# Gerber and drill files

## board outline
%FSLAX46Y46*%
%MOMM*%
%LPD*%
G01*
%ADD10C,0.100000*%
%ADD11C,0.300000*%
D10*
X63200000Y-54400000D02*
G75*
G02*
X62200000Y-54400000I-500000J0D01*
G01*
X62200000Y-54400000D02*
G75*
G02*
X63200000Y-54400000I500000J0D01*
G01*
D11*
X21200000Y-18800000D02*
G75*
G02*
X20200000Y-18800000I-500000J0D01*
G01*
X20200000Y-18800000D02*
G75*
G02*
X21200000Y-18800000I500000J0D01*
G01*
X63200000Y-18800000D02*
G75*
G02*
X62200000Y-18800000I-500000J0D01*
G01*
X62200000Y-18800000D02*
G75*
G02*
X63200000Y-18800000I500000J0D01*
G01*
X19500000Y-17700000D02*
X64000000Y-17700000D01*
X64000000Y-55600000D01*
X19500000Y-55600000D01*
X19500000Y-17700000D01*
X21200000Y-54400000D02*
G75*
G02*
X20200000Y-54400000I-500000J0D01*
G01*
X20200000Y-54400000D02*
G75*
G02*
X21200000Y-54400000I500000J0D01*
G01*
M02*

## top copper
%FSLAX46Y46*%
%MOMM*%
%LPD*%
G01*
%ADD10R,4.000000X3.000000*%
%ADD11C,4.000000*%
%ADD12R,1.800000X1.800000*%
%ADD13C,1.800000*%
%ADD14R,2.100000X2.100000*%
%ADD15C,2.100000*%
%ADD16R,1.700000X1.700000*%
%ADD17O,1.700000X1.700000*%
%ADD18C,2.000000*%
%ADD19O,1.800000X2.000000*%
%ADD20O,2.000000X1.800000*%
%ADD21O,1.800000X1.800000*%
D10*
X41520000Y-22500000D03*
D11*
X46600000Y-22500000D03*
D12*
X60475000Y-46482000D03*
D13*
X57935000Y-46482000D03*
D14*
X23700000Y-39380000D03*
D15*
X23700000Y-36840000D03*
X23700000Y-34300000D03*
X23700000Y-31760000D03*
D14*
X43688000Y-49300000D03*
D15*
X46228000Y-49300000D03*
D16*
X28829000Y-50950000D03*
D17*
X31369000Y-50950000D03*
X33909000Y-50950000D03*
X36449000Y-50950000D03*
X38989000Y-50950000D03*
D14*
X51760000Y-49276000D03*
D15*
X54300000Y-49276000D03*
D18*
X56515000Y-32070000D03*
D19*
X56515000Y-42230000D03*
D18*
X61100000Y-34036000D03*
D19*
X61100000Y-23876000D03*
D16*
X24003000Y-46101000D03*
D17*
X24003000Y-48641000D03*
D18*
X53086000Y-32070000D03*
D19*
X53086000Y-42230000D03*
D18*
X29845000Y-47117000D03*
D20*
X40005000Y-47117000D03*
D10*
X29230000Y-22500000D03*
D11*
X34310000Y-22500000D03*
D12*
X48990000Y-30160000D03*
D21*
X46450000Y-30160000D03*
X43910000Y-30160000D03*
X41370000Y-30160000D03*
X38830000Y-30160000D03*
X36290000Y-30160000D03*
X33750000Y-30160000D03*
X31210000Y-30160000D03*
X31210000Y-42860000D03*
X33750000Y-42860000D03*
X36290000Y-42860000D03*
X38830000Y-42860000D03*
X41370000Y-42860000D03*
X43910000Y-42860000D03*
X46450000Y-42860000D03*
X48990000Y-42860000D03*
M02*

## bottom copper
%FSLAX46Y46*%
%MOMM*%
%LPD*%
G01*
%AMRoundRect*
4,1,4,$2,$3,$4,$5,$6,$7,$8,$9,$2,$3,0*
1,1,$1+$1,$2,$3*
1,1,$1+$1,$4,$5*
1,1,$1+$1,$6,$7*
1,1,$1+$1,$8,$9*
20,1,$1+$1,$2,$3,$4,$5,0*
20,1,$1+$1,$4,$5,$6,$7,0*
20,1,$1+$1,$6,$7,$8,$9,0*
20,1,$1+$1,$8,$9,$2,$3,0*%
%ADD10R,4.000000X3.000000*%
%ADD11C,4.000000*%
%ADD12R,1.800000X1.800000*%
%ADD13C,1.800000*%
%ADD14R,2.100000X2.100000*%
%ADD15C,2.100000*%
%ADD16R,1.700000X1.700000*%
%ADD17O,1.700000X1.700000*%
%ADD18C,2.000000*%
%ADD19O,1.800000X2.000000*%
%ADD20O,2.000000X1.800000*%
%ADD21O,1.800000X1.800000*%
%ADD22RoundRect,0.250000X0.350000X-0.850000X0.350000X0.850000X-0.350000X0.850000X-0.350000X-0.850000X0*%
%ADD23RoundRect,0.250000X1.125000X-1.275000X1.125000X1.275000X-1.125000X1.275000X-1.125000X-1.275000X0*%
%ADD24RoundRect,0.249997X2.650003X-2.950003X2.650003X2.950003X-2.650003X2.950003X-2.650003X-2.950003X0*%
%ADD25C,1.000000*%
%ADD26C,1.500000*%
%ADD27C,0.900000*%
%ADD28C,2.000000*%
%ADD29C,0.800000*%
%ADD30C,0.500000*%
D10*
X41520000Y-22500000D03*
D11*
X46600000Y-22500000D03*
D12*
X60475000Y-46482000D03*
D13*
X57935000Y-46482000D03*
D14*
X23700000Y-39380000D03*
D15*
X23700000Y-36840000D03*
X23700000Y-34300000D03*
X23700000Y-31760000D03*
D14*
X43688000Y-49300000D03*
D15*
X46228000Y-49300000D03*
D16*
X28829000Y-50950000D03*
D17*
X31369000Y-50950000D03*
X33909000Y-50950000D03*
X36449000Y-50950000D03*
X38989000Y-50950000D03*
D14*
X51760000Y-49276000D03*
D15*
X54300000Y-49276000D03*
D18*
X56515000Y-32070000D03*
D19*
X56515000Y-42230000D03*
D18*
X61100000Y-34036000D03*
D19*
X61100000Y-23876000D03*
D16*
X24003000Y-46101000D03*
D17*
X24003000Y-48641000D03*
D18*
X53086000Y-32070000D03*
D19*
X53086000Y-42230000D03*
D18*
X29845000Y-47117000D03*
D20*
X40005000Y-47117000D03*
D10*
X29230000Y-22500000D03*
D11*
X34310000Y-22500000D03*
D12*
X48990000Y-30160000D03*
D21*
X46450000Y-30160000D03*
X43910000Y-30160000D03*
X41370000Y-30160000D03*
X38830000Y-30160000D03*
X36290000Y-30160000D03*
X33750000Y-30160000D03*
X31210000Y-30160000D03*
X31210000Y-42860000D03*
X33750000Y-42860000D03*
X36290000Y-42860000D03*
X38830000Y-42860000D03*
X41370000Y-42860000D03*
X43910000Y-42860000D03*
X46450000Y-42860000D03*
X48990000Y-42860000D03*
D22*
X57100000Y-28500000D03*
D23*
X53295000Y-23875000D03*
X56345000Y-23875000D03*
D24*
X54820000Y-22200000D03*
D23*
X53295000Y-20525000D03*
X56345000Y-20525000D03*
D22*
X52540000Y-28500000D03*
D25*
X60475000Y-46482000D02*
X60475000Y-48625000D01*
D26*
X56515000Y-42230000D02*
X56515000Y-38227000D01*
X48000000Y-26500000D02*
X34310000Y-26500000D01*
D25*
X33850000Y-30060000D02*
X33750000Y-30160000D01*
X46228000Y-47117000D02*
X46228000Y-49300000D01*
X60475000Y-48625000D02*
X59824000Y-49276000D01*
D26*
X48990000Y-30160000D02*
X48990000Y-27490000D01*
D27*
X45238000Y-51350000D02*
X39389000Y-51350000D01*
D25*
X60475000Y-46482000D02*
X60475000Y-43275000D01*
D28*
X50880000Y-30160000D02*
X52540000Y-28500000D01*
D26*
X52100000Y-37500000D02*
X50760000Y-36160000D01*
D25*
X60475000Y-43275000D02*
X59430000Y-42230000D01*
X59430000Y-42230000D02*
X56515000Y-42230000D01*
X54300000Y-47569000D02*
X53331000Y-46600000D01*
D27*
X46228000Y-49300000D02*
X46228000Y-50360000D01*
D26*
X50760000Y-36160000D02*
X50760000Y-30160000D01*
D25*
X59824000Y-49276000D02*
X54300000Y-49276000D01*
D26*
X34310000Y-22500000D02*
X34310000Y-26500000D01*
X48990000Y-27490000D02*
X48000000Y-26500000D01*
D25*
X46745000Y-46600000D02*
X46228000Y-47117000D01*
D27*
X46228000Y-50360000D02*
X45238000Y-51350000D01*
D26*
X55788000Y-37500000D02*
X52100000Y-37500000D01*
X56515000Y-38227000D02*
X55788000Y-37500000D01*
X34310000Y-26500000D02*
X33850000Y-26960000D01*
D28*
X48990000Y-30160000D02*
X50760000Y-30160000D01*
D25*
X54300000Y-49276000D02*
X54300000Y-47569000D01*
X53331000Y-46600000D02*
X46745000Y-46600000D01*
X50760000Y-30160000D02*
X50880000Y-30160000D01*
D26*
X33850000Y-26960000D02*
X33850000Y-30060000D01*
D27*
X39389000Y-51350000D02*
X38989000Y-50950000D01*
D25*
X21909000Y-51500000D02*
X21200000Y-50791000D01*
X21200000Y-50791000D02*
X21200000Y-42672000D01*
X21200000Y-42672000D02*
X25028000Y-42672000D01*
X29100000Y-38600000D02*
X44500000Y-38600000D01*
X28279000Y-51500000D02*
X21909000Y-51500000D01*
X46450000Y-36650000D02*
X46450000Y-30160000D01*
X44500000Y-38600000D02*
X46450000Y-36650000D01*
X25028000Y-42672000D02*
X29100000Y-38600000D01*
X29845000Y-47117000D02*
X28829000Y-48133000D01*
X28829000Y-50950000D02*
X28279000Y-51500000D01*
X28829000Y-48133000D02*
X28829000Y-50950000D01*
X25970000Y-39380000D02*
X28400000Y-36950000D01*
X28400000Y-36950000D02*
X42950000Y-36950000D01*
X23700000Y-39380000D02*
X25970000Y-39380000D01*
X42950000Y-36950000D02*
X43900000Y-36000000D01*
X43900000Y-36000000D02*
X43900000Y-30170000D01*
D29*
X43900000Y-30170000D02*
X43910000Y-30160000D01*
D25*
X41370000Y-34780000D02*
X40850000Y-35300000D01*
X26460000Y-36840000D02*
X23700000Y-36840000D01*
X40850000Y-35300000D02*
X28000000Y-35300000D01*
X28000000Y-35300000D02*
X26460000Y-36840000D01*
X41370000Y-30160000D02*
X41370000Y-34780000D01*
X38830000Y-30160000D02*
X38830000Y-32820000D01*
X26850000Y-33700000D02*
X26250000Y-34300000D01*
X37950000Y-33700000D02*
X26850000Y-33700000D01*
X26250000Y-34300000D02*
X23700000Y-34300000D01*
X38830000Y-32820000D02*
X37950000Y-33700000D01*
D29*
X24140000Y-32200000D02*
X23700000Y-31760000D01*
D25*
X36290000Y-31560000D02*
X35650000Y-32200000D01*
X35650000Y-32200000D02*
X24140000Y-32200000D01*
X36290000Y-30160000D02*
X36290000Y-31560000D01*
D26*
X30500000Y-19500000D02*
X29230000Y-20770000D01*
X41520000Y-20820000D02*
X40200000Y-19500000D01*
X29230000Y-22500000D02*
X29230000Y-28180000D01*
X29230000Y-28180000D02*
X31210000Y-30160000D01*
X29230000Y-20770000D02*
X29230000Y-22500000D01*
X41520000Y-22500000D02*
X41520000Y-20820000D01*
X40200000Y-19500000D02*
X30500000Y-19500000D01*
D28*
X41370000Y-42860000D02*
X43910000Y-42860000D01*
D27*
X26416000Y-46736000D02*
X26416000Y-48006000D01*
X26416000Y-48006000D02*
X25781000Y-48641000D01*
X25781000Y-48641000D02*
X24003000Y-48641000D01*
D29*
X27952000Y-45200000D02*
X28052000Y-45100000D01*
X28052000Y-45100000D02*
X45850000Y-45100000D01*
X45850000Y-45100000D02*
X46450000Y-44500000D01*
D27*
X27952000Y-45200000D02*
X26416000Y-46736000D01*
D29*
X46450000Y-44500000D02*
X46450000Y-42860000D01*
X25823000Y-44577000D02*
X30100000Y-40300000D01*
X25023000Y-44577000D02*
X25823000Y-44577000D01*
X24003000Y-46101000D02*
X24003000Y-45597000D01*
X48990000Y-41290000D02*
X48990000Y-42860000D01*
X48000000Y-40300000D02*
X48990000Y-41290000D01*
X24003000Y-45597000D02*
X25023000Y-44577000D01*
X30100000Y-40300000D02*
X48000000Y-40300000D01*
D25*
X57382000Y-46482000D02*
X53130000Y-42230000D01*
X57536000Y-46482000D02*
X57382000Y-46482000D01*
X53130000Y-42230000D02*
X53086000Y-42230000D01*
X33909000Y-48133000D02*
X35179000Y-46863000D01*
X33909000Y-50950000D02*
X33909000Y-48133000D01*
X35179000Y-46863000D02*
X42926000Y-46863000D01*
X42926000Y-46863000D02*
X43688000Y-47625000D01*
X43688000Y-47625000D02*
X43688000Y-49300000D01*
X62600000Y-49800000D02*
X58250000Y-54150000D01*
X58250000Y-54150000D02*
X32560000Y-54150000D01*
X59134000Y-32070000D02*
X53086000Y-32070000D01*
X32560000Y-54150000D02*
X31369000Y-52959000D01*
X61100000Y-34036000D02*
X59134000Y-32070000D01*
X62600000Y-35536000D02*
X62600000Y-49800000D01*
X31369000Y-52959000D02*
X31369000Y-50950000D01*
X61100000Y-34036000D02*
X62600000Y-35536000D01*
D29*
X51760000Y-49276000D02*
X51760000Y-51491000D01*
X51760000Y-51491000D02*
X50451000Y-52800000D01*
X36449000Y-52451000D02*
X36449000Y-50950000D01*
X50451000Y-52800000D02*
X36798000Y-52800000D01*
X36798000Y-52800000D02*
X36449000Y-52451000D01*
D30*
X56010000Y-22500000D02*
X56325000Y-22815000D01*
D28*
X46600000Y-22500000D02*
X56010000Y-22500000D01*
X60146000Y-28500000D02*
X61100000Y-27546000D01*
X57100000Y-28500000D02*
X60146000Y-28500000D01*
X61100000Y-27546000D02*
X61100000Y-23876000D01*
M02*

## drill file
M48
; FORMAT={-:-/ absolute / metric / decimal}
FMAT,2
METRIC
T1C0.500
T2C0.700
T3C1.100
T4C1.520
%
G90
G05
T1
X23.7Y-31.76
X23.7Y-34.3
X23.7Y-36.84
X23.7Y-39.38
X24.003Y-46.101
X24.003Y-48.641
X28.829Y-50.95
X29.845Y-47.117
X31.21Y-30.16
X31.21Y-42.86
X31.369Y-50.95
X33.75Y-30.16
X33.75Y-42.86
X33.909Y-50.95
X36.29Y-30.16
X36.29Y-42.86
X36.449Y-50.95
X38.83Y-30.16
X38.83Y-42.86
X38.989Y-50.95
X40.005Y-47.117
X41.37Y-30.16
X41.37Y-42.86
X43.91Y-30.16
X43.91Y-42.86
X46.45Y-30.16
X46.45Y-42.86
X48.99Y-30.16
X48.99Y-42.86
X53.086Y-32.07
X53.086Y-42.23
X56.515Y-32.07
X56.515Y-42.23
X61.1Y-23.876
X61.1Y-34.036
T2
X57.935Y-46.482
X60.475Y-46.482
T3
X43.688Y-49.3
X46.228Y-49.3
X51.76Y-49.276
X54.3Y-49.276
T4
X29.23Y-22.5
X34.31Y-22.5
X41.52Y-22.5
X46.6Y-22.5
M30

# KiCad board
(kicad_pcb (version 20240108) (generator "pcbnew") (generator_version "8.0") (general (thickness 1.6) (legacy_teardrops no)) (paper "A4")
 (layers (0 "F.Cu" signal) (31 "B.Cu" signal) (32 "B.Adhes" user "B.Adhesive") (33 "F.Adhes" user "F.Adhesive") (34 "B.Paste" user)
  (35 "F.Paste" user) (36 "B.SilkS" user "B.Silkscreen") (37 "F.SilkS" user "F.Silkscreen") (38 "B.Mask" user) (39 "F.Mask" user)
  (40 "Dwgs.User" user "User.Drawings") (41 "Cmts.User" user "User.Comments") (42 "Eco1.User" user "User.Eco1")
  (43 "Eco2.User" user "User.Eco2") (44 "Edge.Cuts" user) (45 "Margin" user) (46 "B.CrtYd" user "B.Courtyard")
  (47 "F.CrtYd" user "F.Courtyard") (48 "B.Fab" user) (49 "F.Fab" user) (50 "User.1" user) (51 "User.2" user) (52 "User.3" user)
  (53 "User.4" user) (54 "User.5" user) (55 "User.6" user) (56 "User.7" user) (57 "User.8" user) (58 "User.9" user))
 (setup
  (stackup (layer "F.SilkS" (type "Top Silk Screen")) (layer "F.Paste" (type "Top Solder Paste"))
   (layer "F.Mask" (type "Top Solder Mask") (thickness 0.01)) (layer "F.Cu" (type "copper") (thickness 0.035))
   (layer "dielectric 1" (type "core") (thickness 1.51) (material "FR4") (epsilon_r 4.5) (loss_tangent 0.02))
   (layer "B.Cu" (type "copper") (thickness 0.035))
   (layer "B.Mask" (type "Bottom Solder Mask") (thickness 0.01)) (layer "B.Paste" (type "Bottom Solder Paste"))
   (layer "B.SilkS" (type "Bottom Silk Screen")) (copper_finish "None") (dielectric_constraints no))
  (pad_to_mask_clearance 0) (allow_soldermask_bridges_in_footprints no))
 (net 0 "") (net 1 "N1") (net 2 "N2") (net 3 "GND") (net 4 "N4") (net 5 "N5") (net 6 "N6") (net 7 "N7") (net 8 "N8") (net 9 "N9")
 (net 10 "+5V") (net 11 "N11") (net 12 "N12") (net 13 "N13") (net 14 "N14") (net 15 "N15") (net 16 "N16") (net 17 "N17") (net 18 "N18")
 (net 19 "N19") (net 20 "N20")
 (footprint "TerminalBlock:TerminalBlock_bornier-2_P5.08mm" (layer "F.Cu") (at 41.52 22.5)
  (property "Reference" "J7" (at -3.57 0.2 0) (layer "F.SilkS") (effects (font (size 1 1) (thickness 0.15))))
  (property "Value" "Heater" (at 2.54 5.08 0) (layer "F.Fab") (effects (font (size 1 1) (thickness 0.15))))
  (pad "1" thru_hole rect (at 0 0) (size 4 3) (drill 1.52) (layers "*.Cu" "*.Mask") (remove_unused_layers no) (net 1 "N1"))
  (pad "2" thru_hole circle (at 5.08 0) (size 4 3) (drill 1.52) (layers "*.Cu" "*.Mask") (remove_unused_layers no) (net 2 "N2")))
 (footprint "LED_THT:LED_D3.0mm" (layer "F.Cu") (at 60.475 46.482 180)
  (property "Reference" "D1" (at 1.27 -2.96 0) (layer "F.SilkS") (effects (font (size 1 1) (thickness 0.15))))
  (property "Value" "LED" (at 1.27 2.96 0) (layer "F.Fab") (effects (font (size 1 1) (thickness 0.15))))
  (pad "1" thru_hole rect (at 0 0 180) (size 1.8 1.8) (drill 0.7) (layers "*.Cu" "*.Mask") (remove_unused_layers no) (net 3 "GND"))
  (pad "2" thru_hole circle (at 2.54 0 180) (size 1.8 1.8) (drill 0.7) (layers "*.Cu" "*.Mask") (remove_unused_layers no) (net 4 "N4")))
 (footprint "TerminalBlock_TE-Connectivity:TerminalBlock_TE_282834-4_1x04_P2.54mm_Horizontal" (layer "F.Cu") (at 23.7 39.38 90)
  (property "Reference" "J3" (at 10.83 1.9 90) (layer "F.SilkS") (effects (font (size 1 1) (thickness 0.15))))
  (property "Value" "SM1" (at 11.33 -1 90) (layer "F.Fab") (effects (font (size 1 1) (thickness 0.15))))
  (pad "1" thru_hole rect (at 0 0 90) (size 2.1 2.1) (drill 0.5) (layers "*.Cu" "*.Mask") (remove_unused_layers no) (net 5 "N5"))
  (pad "2" thru_hole circle (at 2.54 0 90) (size 2.1 2.1) (drill 0.5) (layers "*.Cu" "*.Mask") (remove_unused_layers no) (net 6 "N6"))
  (pad "3" thru_hole circle (at 5.08 0 90) (size 2.1 2.1) (drill 0.5) (layers "*.Cu" "*.Mask") (remove_unused_layers no) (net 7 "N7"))
  (pad "4" thru_hole circle (at 7.62 0 90) (size 2.1 2.1) (drill 0.5) (layers "*.Cu" "*.Mask") (remove_unused_layers no) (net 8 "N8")))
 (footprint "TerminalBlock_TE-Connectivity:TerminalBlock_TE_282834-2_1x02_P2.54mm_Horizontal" (layer "F.Cu") (at 43.688 49.3)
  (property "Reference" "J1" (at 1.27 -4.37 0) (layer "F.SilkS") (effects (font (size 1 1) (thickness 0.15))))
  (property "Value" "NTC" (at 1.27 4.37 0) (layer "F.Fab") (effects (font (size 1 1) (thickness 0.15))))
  (pad "1" thru_hole rect (at 0 0) (size 2.1 2.1) (drill 1.1) (layers "*.Cu" "*.Mask") (remove_unused_layers no) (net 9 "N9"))
  (pad "2" thru_hole circle (at 2.54 0) (size 2.1 2.1) (drill 1.1) (layers "*.Cu" "*.Mask") (remove_unused_layers no) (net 3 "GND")))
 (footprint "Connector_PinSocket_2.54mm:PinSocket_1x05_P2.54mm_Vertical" (layer "F.Cu") (at 28.829 50.95 90)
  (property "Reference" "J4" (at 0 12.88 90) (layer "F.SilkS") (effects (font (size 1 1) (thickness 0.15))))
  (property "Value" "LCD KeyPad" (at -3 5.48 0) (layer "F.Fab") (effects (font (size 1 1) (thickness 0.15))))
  (pad "1" thru_hole rect (at 0 0 90) (size 1.7 1.7) (drill 0.5) (layers "*.Cu" "*.Mask") (remove_unused_layers no) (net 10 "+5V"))
  (pad "2" thru_hole oval (at 0 2.54 90) (size 1.7 1.7) (drill 0.5) (layers "*.Cu" "*.Mask") (remove_unused_layers no) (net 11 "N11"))
  (pad "3" thru_hole oval (at 0 5.08 90) (size 1.7 1.7) (drill 0.5) (layers "*.Cu" "*.Mask") (remove_unused_layers no) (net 9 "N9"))
  (pad "4" thru_hole oval (at 0 7.62 90) (size 1.7 1.7) (drill 0.5) (layers "*.Cu" "*.Mask") (remove_unused_layers no) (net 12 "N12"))
  (pad "5" thru_hole oval (at 0 10.16 90) (size 1.7 1.7) (drill 0.5) (layers "*.Cu" "*.Mask") (remove_unused_layers no) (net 3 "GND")))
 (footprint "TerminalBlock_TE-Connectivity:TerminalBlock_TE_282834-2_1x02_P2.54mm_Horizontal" (layer "F.Cu") (at 51.76 49.276)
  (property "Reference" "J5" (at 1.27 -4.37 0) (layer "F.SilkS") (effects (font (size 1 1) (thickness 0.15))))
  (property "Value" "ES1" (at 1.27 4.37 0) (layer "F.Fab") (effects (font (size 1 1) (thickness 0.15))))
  (pad "1" thru_hole rect (at 0 0) (size 2.1 2.1) (drill 1.1) (layers "*.Cu" "*.Mask") (remove_unused_layers no) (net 12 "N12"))
  (pad "2" thru_hole circle (at 2.54 0) (size 2.1 2.1) (drill 1.1) (layers "*.Cu" "*.Mask") (remove_unused_layers no) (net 3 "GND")))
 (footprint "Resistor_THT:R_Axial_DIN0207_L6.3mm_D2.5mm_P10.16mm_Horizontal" (layer "F.Cu") (at 56.515 32.07 -90)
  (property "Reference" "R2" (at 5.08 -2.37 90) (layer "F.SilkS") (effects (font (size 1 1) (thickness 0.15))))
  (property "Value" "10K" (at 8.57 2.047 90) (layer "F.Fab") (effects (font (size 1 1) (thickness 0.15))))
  (pad "1" thru_hole circle (at 0 0 270) (size 2 1.6) (drill 0.5) (layers "*.Cu" "*.Mask") (remove_unused_layers no) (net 11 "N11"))
  (pad "2" thru_hole oval (at 10.16 0 270) (size 2 1.8) (drill 0.5) (layers "*.Cu" "*.Mask") (remove_unused_layers no) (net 3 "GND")))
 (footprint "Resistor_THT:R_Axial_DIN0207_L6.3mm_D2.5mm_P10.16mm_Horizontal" (layer "F.Cu") (at 61.1 34.036 90)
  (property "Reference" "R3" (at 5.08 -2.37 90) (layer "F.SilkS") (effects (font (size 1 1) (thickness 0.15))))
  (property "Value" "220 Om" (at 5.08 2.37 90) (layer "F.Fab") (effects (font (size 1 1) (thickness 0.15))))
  (pad "1" thru_hole circle (at 0 0 90) (size 2 1.6) (drill 0.5) (layers "*.Cu" "*.Mask") (remove_unused_layers no) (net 11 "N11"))
  (pad "2" thru_hole oval (at 10.16 0 90) (size 2 1.8) (drill 0.5) (layers "*.Cu" "*.Mask") (remove_unused_layers no) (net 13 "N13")))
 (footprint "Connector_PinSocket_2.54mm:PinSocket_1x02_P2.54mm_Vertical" (layer "F.Cu") (at 24.003 46.101)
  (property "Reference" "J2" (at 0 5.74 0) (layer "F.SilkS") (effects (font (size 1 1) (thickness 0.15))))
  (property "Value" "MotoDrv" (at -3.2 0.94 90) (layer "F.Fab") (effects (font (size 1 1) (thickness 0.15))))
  (pad "1" thru_hole rect (at 0 0) (size 1.7 1.7) (drill 0.5) (layers "*.Cu" "*.Mask") (remove_unused_layers no) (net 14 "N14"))
  (pad "2" thru_hole oval (at 0 2.54) (size 1.7 1.7) (drill 0.5) (layers "*.Cu" "*.Mask") (remove_unused_layers no) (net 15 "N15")))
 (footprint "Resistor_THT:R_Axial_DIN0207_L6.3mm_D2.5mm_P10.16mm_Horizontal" (layer "F.Cu") (at 53.086 32.07 -90)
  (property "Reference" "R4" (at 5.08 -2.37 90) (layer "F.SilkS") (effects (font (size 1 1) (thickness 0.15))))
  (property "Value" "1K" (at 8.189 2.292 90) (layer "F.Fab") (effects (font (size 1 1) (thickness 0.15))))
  (pad "1" thru_hole circle (at 0 0 270) (size 2 1.6) (drill 0.5) (layers "*.Cu" "*.Mask") (remove_unused_layers no) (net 11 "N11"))
  (pad "2" thru_hole oval (at 10.16 0 270) (size 2 1.8) (drill 0.5) (layers "*.Cu" "*.Mask") (remove_unused_layers no) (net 4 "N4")))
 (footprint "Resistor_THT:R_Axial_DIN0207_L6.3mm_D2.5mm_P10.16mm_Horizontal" (layer "F.Cu") (at 29.845 47.117)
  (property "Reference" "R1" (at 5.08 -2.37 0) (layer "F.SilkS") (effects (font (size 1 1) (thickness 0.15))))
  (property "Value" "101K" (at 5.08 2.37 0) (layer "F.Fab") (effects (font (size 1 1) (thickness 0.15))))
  (pad "1" thru_hole circle (at 0 0) (size 2 1.6) (drill 0.5) (layers "*.Cu" "*.Mask") (remove_unused_layers no) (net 10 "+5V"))
  (pad "2" thru_hole oval (at 10.16 0) (size 2 1.8) (drill 0.5) (layers "*.Cu" "*.Mask") (remove_unused_layers no) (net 9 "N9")))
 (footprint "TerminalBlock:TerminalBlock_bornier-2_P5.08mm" (layer "F.Cu") (at 29.23 22.5)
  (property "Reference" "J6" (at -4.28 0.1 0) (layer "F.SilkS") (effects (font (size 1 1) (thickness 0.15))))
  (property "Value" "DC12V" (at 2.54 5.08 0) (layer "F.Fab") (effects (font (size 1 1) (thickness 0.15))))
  (pad "1" thru_hole rect (at 0 0) (size 4 3) (drill 1.52) (layers "*.Cu" "*.Mask") (remove_unused_layers no) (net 1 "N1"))
  (pad "2" thru_hole circle (at 5.08 0) (size 4 3) (drill 1.52) (layers "*.Cu" "*.Mask") (remove_unused_layers no) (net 3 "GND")))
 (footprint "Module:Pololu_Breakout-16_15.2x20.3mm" (layer "F.Cu") (at 48.99 30.16 -90)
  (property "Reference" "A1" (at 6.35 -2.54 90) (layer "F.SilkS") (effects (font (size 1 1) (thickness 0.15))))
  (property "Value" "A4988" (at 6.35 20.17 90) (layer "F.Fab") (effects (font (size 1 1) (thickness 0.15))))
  (pad "1" thru_hole rect (at 0 0 270) (size 1.8 1.8) (drill 0.5) (layers "*.Cu" "*.Mask") (remove_unused_layers no) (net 3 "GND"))
  (pad "2" thru_hole oval (at 0 2.54 270) (size 1.8 1.8) (drill 0.5) (layers "*.Cu" "*.Mask") (remove_unused_layers no) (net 10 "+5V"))
  (pad "3" thru_hole oval (at 0 5.08 270) (size 1.8 1.8) (drill 0.5) (layers "*.Cu" "*.Mask") (remove_unused_layers no) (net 5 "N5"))
  (pad "4" thru_hole oval (at 0 7.62 270) (size 1.8 1.8) (drill 0.5) (layers "*.Cu" "*.Mask") (remove_unused_layers no) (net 6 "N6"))
  (pad "5" thru_hole oval (at 0 10.16 270) (size 1.8 1.8) (drill 0.5) (layers "*.Cu" "*.Mask") (remove_unused_layers no) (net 7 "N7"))
  (pad "6" thru_hole oval (at 0 12.7 270) (size 1.8 1.8) (drill 0.5) (layers "*.Cu" "*.Mask") (remove_unused_layers no) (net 8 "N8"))
  (pad "7" thru_hole oval (at 0 15.24 270) (size 1.8 1.8) (drill 0.5) (layers "*.Cu" "*.Mask") (remove_unused_layers no) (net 3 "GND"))
  (pad "8" thru_hole oval (at 0 17.78 270) (size 1.8 1.8) (drill 0.5) (layers "*.Cu" "*.Mask") (remove_unused_layers no) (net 1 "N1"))
  (pad "9" thru_hole oval (at 12.7 17.78 270) (size 1.8 1.8) (drill 0.5) (layers "*.Cu" "*.Mask") (remove_unused_layers no) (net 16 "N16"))
  (pad "10" thru_hole oval (at 12.7 15.24 270) (size 1.8 1.8) (drill 0.5) (layers "*.Cu" "*.Mask") (remove_unused_layers no) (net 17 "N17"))
  (pad "11" thru_hole oval (at 12.7 12.7 270) (size 1.8 1.8) (drill 0.5) (layers "*.Cu" "*.Mask") (remove_unused_layers no) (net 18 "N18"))
  (pad "12" thru_hole oval (at 12.7 10.16 270) (size 1.8 1.8) (drill 0.5) (layers "*.Cu" "*.Mask") (remove_unused_layers no) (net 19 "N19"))
  (pad "13" thru_hole oval (at 12.7 7.62 270) (size 1.8 1.8) (drill 0.5) (layers "*.Cu" "*.Mask") (remove_unused_layers no) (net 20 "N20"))
  (pad "14" thru_hole oval (at 12.7 5.08 270) (size 1.8 1.8) (drill 0.5) (layers "*.Cu" "*.Mask") (remove_unused_layers no) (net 20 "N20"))
  (pad "15" thru_hole oval (at 12.7 2.54 270) (size 1.8 1.8) (drill 0.5) (layers "*.Cu" "*.Mask") (remove_unused_layers no) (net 15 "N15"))
  (pad "16" thru_hole oval (at 12.7 0 270) (size 1.8 1.8) (drill 0.5) (layers "*.Cu" "*.Mask") (remove_unused_layers no) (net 14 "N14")))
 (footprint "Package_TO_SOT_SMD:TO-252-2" (layer "B.Cu") (at 54.82 23.46 90)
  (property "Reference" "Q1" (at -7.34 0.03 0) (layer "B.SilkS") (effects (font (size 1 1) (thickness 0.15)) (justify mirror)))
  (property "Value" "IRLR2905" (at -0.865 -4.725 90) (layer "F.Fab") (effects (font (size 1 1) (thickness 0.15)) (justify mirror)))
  (pad "1" smd roundrect (at -5.04 2.28 90) (size 2.2 1.2) (layers "B.Cu" "B.Paste" "B.Mask") (roundrect_rratio 0.208333) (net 13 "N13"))
  (pad "2" smd roundrect (at -0.415 -1.525 90) (size 3.05 2.75) (layers "B.Cu" "B.Paste") (roundrect_rratio 0.090909) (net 2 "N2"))
  (pad "2" smd roundrect (at -0.415 1.525 90) (size 3.05 2.75) (layers "B.Cu" "B.Paste") (roundrect_rratio 0.090909) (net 2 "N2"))
  (pad "2" smd roundrect (at 1.26 0 90) (size 6.4 5.8) (layers "B.Cu" "B.Mask") (roundrect_rratio 0.043103) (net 2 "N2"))
  (pad "2" smd roundrect (at 2.935 -1.525 90) (size 3.05 2.75) (layers "B.Cu" "B.Paste") (roundrect_rratio 0.090909) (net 2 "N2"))
  (pad "2" smd roundrect (at 2.935 1.525 90) (size 3.05 2.75) (layers "B.Cu" "B.Paste") (roundrect_rratio 0.090909) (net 2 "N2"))
  (pad "3" smd roundrect (at -5.04 -2.28 90) (size 2.2 1.2) (layers "B.Cu" "B.Paste" "B.Mask") (roundrect_rratio 0.208333) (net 3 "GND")))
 (gr_circle (center 62.7 54.4) (end 63.2 54.4) (stroke (width 0.1) (type default)) (fill none) (layer "Edge.Cuts"))
 (gr_circle (center 20.7 18.8) (end 21.2 18.8) (stroke (width 0.3) (type default)) (fill none) (layer "Edge.Cuts"))
 (gr_circle (center 62.7 18.8) (end 63.2 18.8) (stroke (width 0.3) (type default)) (fill none) (layer "Edge.Cuts"))
 (gr_rect (start 19.5 17.7) (end 64 55.6) (stroke (width 0.3) (type default)) (fill none) (layer "Edge.Cuts"))
 (gr_circle (center 20.7 54.4) (end 21.2 54.4) (stroke (width 0.3) (type default)) (fill none) (layer "Edge.Cuts"))
 (segment (start 60.475 46.482) (end 60.475 48.625) (width 1) (layer "B.Cu") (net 3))
 (segment (start 56.515 42.23) (end 56.515 38.227) (width 1.5) (layer "B.Cu") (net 3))
 (segment (start 48 26.5) (end 34.31 26.5) (width 1.5) (layer "B.Cu") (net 3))
 (segment (start 33.85 30.06) (end 33.75 30.16) (width 1) (layer "B.Cu") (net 3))
 (segment (start 46.228 47.117) (end 46.228 49.3) (width 1) (layer "B.Cu") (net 3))
 (segment (start 60.475 48.625) (end 59.824 49.276) (width 1) (layer "B.Cu") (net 3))
 (segment (start 48.99 30.16) (end 48.99 27.49) (width 1.5) (layer "B.Cu") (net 3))
 (segment (start 45.238 51.35) (end 39.389 51.35) (width 0.9) (layer "B.Cu") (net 3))
 (segment (start 60.475 46.482) (end 60.475 43.275) (width 1) (layer "B.Cu") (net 3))
 (segment (start 50.88 30.16) (end 52.54 28.5) (width 2) (layer "B.Cu") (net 3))
 (segment (start 52.1 37.5) (end 50.76 36.16) (width 1.5) (layer "B.Cu") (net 3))
 (segment (start 60.475 43.275) (end 59.43 42.23) (width 1) (layer "B.Cu") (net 3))
 (segment (start 59.43 42.23) (end 56.515 42.23) (width 1) (layer "B.Cu") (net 3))
 (segment (start 54.3 47.569) (end 53.331 46.6) (width 1) (layer "B.Cu") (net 3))
 (segment (start 46.228 49.3) (end 46.228 50.36) (width 0.9) (layer "B.Cu") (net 3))
 (segment (start 50.76 36.16) (end 50.76 30.16) (width 1.5) (layer "B.Cu") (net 3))
 (segment (start 59.824 49.276) (end 54.3 49.276) (width 1) (layer "B.Cu") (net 3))
 (segment (start 34.31 22.5) (end 34.31 26.5) (width 1.5) (layer "B.Cu") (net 3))
 (segment (start 48.99 27.49) (end 48 26.5) (width 1.5) (layer "B.Cu") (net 3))
 (segment (start 46.745 46.6) (end 46.228 47.117) (width 1) (layer "B.Cu") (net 3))
 (segment (start 46.228 50.36) (end 45.238 51.35) (width 0.9) (layer "B.Cu") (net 3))
 (segment (start 55.788 37.5) (end 52.1 37.5) (width 1.5) (layer "B.Cu") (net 3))
 (segment (start 56.515 38.227) (end 55.788 37.5) (width 1.5) (layer "B.Cu") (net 3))
 (segment (start 34.31 26.5) (end 33.85 26.96) (width 1.5) (layer "B.Cu") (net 3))
 (segment (start 48.99 30.16) (end 50.76 30.16) (width 2) (layer "B.Cu") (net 3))
 (segment (start 54.3 49.276) (end 54.3 47.569) (width 1) (layer "B.Cu") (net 3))
 (segment (start 53.331 46.6) (end 46.745 46.6) (width 1) (layer "B.Cu") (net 3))
 (segment (start 50.76 30.16) (end 50.88 30.16) (width 1) (layer "B.Cu") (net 3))
 (segment (start 33.85 26.96) (end 33.85 30.06) (width 1.5) (layer "B.Cu") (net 3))
 (segment (start 39.389 51.35) (end 38.989 50.95) (width 0.9) (layer "B.Cu") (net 3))
 (segment (start 21.909 51.5) (end 21.2 50.791) (width 1) (layer "B.Cu") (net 10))
 (segment (start 21.2 50.791) (end 21.2 42.672) (width 1) (layer "B.Cu") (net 10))
 (segment (start 21.2 42.672) (end 25.028 42.672) (width 1) (layer "B.Cu") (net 10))
 (segment (start 29.1 38.6) (end 44.5 38.6) (width 1) (layer "B.Cu") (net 10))
 (segment (start 28.279 51.5) (end 21.909 51.5) (width 1) (layer "B.Cu") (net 10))
 (segment (start 46.45 36.65) (end 46.45 30.16) (width 1) (layer "B.Cu") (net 10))
 (segment (start 44.5 38.6) (end 46.45 36.65) (width 1) (layer "B.Cu") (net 10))
 (segment (start 25.028 42.672) (end 29.1 38.6) (width 1) (layer "B.Cu") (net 10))
 (segment (start 29.845 47.117) (end 28.829 48.133) (width 1) (layer "B.Cu") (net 10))
 (segment (start 28.829 50.95) (end 28.279 51.5) (width 1) (layer "B.Cu") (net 10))
 (segment (start 28.829 48.133) (end 28.829 50.95) (width 1) (layer "B.Cu") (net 10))
 (segment (start 25.97 39.38) (end 28.4 36.95) (width 1) (layer "B.Cu") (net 5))
 (segment (start 28.4 36.95) (end 42.95 36.95) (width 1) (layer "B.Cu") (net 5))
 (segment (start 23.7 39.38) (end 25.97 39.38) (width 1) (layer "B.Cu") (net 5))
 (segment (start 42.95 36.95) (end 43.9 36) (width 1) (layer "B.Cu") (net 5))
 (segment (start 43.9 36) (end 43.9 30.17) (width 1) (layer "B.Cu") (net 5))
 (segment (start 43.9 30.17) (end 43.91 30.16) (width 0.8) (layer "B.Cu") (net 5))
 (segment (start 41.37 34.78) (end 40.85 35.3) (width 1) (layer "B.Cu") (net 6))
 (segment (start 26.46 36.84) (end 23.7 36.84) (width 1) (layer "B.Cu") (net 6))
 (segment (start 40.85 35.3) (end 28 35.3) (width 1) (layer "B.Cu") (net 6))
 (segment (start 28 35.3) (end 26.46 36.84) (width 1) (layer "B.Cu") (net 6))
 (segment (start 41.37 30.16) (end 41.37 34.78) (width 1) (layer "B.Cu") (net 6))
 (segment (start 38.83 30.16) (end 38.83 32.82) (width 1) (layer "B.Cu") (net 7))
 (segment (start 26.85 33.7) (end 26.25 34.3) (width 1) (layer "B.Cu") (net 7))
 (segment (start 37.95 33.7) (end 26.85 33.7) (width 1) (layer "B.Cu") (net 7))
 (segment (start 26.25 34.3) (end 23.7 34.3) (width 1) (layer "B.Cu") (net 7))
 (segment (start 38.83 32.82) (end 37.95 33.7) (width 1) (layer "B.Cu") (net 7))
 (segment (start 24.14 32.2) (end 23.7 31.76) (width 0.8) (layer "B.Cu") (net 8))
 (segment (start 36.29 31.56) (end 35.65 32.2) (width 1) (layer "B.Cu") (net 8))
 (segment (start 35.65 32.2) (end 24.14 32.2) (width 1) (layer "B.Cu") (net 8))
 (segment (start 36.29 30.16) (end 36.29 31.56) (width 1) (layer "B.Cu") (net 8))
 (segment (start 30.5 19.5) (end 29.23 20.77) (width 1.5) (layer "B.Cu") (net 1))
 (segment (start 41.52 20.82) (end 40.2 19.5) (width 1.5) (layer "B.Cu") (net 1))
 (segment (start 29.23 22.5) (end 29.23 28.18) (width 1.5) (layer "B.Cu") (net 1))
 (segment (start 29.23 28.18) (end 31.21 30.16) (width 1.5) (layer "B.Cu") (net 1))
 (segment (start 29.23 20.77) (end 29.23 22.5) (width 1.5) (layer "B.Cu") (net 1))
 (segment (start 41.52 22.5) (end 41.52 20.82) (width 1.5) (layer "B.Cu") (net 1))
 (segment (start 40.2 19.5) (end 30.5 19.5) (width 1.5) (layer "B.Cu") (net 1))
 (segment (start 41.37 42.86) (end 43.91 42.86) (width 2) (layer "B.Cu") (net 20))
 (segment (start 26.416 46.736) (end 26.416 48.006) (width 0.9) (layer "B.Cu") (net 15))
 (segment (start 26.416 48.006) (end 25.781 48.641) (width 0.9) (layer "B.Cu") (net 15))
 (segment (start 25.781 48.641) (end 24.003 48.641) (width 0.9) (layer "B.Cu") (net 15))
 (segment (start 27.952 45.2) (end 28.052 45.1) (width 0.8) (layer "B.Cu") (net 15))
 (segment (start 28.052 45.1) (end 45.85 45.1) (width 0.8) (layer "B.Cu") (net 15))
 (segment (start 45.85 45.1) (end 46.45 44.5) (width 0.8) (layer "B.Cu") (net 15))
 (segment (start 27.952 45.2) (end 26.416 46.736) (width 0.9) (layer "B.Cu") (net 15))
 (segment (start 46.45 44.5) (end 46.45 42.86) (width 0.8) (layer "B.Cu") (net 15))
 (segment (start 25.823 44.577) (end 30.1 40.3) (width 0.8) (layer "B.Cu") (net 14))
 (segment (start 25.023 44.577) (end 25.823 44.577) (width 0.8) (layer "B.Cu") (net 14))
 (segment (start 24.003 46.101) (end 24.003 45.597) (width 0.8) (layer "B.Cu") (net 14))
 (segment (start 48.99 41.29) (end 48.99 42.86) (width 0.8) (layer "B.Cu") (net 14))
 (segment (start 48 40.3) (end 48.99 41.29) (width 0.8) (layer "B.Cu") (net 14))
 (segment (start 24.003 45.597) (end 25.023 44.577) (width 0.8) (layer "B.Cu") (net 14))
 (segment (start 30.1 40.3) (end 48 40.3) (width 0.8) (layer "B.Cu") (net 14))
 (segment (start 57.382 46.482) (end 53.13 42.23) (width 1) (layer "B.Cu") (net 4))
 (segment (start 57.536 46.482) (end 57.382 46.482) (width 1) (layer "B.Cu") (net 4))
 (segment (start 53.13 42.23) (end 53.086 42.23) (width 1) (layer "B.Cu") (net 4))
 (segment (start 33.909 48.133) (end 35.179 46.863) (width 1) (layer "B.Cu") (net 9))
 (segment (start 33.909 50.95) (end 33.909 48.133) (width 1) (layer "B.Cu") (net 9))
 (segment (start 35.179 46.863) (end 42.926 46.863) (width 1) (layer "B.Cu") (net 9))
 (segment (start 42.926 46.863) (end 43.688 47.625) (width 1) (layer "B.Cu") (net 9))
 (segment (start 43.688 47.625) (end 43.688 49.3) (width 1) (layer "B.Cu") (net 9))
 (segment (start 62.6 49.8) (end 58.25 54.15) (width 1) (layer "B.Cu") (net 11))
 (segment (start 58.25 54.15) (end 32.56 54.15) (width 1) (layer "B.Cu") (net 11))
 (segment (start 59.134 32.07) (end 53.086 32.07) (width 1) (layer "B.Cu") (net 11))
 (segment (start 32.56 54.15) (end 31.369 52.959) (width 1) (layer "B.Cu") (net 11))
 (segment (start 61.1 34.036) (end 59.134 32.07) (width 1) (layer "B.Cu") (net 11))
 (segment (start 62.6 35.536) (end 62.6 49.8) (width 1) (layer "B.Cu") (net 11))
 (segment (start 31.369 52.959) (end 31.369 50.95) (width 1) (layer "B.Cu") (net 11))
 (segment (start 61.1 34.036) (end 62.6 35.536) (width 1) (layer "B.Cu") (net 11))
 (segment (start 51.76 49.276) (end 51.76 51.491) (width 0.8) (layer "B.Cu") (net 12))
 (segment (start 51.76 51.491) (end 50.451 52.8) (width 0.8) (layer "B.Cu") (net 12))
 (segment (start 36.449 52.451) (end 36.449 50.95) (width 0.8) (layer "B.Cu") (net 12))
 (segment (start 50.451 52.8) (end 36.798 52.8) (width 0.8) (layer "B.Cu") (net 12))
 (segment (start 36.798 52.8) (end 36.449 52.451) (width 0.8) (layer "B.Cu") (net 12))
 (segment (start 56.01 22.5) (end 56.325 22.815) (width 0.5) (layer "B.Cu") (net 2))
 (segment (start 46.6 22.5) (end 56.01 22.5) (width 2) (layer "B.Cu") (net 2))
 (segment (start 60.146 28.5) (end 61.1 27.546) (width 2) (layer "B.Cu") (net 13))
 (segment (start 57.1 28.5) (end 60.146 28.5) (width 2) (layer "B.Cu") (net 13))
 (segment (start 61.1 27.546) (end 61.1 23.876) (width 2) (layer "B.Cu") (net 13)))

